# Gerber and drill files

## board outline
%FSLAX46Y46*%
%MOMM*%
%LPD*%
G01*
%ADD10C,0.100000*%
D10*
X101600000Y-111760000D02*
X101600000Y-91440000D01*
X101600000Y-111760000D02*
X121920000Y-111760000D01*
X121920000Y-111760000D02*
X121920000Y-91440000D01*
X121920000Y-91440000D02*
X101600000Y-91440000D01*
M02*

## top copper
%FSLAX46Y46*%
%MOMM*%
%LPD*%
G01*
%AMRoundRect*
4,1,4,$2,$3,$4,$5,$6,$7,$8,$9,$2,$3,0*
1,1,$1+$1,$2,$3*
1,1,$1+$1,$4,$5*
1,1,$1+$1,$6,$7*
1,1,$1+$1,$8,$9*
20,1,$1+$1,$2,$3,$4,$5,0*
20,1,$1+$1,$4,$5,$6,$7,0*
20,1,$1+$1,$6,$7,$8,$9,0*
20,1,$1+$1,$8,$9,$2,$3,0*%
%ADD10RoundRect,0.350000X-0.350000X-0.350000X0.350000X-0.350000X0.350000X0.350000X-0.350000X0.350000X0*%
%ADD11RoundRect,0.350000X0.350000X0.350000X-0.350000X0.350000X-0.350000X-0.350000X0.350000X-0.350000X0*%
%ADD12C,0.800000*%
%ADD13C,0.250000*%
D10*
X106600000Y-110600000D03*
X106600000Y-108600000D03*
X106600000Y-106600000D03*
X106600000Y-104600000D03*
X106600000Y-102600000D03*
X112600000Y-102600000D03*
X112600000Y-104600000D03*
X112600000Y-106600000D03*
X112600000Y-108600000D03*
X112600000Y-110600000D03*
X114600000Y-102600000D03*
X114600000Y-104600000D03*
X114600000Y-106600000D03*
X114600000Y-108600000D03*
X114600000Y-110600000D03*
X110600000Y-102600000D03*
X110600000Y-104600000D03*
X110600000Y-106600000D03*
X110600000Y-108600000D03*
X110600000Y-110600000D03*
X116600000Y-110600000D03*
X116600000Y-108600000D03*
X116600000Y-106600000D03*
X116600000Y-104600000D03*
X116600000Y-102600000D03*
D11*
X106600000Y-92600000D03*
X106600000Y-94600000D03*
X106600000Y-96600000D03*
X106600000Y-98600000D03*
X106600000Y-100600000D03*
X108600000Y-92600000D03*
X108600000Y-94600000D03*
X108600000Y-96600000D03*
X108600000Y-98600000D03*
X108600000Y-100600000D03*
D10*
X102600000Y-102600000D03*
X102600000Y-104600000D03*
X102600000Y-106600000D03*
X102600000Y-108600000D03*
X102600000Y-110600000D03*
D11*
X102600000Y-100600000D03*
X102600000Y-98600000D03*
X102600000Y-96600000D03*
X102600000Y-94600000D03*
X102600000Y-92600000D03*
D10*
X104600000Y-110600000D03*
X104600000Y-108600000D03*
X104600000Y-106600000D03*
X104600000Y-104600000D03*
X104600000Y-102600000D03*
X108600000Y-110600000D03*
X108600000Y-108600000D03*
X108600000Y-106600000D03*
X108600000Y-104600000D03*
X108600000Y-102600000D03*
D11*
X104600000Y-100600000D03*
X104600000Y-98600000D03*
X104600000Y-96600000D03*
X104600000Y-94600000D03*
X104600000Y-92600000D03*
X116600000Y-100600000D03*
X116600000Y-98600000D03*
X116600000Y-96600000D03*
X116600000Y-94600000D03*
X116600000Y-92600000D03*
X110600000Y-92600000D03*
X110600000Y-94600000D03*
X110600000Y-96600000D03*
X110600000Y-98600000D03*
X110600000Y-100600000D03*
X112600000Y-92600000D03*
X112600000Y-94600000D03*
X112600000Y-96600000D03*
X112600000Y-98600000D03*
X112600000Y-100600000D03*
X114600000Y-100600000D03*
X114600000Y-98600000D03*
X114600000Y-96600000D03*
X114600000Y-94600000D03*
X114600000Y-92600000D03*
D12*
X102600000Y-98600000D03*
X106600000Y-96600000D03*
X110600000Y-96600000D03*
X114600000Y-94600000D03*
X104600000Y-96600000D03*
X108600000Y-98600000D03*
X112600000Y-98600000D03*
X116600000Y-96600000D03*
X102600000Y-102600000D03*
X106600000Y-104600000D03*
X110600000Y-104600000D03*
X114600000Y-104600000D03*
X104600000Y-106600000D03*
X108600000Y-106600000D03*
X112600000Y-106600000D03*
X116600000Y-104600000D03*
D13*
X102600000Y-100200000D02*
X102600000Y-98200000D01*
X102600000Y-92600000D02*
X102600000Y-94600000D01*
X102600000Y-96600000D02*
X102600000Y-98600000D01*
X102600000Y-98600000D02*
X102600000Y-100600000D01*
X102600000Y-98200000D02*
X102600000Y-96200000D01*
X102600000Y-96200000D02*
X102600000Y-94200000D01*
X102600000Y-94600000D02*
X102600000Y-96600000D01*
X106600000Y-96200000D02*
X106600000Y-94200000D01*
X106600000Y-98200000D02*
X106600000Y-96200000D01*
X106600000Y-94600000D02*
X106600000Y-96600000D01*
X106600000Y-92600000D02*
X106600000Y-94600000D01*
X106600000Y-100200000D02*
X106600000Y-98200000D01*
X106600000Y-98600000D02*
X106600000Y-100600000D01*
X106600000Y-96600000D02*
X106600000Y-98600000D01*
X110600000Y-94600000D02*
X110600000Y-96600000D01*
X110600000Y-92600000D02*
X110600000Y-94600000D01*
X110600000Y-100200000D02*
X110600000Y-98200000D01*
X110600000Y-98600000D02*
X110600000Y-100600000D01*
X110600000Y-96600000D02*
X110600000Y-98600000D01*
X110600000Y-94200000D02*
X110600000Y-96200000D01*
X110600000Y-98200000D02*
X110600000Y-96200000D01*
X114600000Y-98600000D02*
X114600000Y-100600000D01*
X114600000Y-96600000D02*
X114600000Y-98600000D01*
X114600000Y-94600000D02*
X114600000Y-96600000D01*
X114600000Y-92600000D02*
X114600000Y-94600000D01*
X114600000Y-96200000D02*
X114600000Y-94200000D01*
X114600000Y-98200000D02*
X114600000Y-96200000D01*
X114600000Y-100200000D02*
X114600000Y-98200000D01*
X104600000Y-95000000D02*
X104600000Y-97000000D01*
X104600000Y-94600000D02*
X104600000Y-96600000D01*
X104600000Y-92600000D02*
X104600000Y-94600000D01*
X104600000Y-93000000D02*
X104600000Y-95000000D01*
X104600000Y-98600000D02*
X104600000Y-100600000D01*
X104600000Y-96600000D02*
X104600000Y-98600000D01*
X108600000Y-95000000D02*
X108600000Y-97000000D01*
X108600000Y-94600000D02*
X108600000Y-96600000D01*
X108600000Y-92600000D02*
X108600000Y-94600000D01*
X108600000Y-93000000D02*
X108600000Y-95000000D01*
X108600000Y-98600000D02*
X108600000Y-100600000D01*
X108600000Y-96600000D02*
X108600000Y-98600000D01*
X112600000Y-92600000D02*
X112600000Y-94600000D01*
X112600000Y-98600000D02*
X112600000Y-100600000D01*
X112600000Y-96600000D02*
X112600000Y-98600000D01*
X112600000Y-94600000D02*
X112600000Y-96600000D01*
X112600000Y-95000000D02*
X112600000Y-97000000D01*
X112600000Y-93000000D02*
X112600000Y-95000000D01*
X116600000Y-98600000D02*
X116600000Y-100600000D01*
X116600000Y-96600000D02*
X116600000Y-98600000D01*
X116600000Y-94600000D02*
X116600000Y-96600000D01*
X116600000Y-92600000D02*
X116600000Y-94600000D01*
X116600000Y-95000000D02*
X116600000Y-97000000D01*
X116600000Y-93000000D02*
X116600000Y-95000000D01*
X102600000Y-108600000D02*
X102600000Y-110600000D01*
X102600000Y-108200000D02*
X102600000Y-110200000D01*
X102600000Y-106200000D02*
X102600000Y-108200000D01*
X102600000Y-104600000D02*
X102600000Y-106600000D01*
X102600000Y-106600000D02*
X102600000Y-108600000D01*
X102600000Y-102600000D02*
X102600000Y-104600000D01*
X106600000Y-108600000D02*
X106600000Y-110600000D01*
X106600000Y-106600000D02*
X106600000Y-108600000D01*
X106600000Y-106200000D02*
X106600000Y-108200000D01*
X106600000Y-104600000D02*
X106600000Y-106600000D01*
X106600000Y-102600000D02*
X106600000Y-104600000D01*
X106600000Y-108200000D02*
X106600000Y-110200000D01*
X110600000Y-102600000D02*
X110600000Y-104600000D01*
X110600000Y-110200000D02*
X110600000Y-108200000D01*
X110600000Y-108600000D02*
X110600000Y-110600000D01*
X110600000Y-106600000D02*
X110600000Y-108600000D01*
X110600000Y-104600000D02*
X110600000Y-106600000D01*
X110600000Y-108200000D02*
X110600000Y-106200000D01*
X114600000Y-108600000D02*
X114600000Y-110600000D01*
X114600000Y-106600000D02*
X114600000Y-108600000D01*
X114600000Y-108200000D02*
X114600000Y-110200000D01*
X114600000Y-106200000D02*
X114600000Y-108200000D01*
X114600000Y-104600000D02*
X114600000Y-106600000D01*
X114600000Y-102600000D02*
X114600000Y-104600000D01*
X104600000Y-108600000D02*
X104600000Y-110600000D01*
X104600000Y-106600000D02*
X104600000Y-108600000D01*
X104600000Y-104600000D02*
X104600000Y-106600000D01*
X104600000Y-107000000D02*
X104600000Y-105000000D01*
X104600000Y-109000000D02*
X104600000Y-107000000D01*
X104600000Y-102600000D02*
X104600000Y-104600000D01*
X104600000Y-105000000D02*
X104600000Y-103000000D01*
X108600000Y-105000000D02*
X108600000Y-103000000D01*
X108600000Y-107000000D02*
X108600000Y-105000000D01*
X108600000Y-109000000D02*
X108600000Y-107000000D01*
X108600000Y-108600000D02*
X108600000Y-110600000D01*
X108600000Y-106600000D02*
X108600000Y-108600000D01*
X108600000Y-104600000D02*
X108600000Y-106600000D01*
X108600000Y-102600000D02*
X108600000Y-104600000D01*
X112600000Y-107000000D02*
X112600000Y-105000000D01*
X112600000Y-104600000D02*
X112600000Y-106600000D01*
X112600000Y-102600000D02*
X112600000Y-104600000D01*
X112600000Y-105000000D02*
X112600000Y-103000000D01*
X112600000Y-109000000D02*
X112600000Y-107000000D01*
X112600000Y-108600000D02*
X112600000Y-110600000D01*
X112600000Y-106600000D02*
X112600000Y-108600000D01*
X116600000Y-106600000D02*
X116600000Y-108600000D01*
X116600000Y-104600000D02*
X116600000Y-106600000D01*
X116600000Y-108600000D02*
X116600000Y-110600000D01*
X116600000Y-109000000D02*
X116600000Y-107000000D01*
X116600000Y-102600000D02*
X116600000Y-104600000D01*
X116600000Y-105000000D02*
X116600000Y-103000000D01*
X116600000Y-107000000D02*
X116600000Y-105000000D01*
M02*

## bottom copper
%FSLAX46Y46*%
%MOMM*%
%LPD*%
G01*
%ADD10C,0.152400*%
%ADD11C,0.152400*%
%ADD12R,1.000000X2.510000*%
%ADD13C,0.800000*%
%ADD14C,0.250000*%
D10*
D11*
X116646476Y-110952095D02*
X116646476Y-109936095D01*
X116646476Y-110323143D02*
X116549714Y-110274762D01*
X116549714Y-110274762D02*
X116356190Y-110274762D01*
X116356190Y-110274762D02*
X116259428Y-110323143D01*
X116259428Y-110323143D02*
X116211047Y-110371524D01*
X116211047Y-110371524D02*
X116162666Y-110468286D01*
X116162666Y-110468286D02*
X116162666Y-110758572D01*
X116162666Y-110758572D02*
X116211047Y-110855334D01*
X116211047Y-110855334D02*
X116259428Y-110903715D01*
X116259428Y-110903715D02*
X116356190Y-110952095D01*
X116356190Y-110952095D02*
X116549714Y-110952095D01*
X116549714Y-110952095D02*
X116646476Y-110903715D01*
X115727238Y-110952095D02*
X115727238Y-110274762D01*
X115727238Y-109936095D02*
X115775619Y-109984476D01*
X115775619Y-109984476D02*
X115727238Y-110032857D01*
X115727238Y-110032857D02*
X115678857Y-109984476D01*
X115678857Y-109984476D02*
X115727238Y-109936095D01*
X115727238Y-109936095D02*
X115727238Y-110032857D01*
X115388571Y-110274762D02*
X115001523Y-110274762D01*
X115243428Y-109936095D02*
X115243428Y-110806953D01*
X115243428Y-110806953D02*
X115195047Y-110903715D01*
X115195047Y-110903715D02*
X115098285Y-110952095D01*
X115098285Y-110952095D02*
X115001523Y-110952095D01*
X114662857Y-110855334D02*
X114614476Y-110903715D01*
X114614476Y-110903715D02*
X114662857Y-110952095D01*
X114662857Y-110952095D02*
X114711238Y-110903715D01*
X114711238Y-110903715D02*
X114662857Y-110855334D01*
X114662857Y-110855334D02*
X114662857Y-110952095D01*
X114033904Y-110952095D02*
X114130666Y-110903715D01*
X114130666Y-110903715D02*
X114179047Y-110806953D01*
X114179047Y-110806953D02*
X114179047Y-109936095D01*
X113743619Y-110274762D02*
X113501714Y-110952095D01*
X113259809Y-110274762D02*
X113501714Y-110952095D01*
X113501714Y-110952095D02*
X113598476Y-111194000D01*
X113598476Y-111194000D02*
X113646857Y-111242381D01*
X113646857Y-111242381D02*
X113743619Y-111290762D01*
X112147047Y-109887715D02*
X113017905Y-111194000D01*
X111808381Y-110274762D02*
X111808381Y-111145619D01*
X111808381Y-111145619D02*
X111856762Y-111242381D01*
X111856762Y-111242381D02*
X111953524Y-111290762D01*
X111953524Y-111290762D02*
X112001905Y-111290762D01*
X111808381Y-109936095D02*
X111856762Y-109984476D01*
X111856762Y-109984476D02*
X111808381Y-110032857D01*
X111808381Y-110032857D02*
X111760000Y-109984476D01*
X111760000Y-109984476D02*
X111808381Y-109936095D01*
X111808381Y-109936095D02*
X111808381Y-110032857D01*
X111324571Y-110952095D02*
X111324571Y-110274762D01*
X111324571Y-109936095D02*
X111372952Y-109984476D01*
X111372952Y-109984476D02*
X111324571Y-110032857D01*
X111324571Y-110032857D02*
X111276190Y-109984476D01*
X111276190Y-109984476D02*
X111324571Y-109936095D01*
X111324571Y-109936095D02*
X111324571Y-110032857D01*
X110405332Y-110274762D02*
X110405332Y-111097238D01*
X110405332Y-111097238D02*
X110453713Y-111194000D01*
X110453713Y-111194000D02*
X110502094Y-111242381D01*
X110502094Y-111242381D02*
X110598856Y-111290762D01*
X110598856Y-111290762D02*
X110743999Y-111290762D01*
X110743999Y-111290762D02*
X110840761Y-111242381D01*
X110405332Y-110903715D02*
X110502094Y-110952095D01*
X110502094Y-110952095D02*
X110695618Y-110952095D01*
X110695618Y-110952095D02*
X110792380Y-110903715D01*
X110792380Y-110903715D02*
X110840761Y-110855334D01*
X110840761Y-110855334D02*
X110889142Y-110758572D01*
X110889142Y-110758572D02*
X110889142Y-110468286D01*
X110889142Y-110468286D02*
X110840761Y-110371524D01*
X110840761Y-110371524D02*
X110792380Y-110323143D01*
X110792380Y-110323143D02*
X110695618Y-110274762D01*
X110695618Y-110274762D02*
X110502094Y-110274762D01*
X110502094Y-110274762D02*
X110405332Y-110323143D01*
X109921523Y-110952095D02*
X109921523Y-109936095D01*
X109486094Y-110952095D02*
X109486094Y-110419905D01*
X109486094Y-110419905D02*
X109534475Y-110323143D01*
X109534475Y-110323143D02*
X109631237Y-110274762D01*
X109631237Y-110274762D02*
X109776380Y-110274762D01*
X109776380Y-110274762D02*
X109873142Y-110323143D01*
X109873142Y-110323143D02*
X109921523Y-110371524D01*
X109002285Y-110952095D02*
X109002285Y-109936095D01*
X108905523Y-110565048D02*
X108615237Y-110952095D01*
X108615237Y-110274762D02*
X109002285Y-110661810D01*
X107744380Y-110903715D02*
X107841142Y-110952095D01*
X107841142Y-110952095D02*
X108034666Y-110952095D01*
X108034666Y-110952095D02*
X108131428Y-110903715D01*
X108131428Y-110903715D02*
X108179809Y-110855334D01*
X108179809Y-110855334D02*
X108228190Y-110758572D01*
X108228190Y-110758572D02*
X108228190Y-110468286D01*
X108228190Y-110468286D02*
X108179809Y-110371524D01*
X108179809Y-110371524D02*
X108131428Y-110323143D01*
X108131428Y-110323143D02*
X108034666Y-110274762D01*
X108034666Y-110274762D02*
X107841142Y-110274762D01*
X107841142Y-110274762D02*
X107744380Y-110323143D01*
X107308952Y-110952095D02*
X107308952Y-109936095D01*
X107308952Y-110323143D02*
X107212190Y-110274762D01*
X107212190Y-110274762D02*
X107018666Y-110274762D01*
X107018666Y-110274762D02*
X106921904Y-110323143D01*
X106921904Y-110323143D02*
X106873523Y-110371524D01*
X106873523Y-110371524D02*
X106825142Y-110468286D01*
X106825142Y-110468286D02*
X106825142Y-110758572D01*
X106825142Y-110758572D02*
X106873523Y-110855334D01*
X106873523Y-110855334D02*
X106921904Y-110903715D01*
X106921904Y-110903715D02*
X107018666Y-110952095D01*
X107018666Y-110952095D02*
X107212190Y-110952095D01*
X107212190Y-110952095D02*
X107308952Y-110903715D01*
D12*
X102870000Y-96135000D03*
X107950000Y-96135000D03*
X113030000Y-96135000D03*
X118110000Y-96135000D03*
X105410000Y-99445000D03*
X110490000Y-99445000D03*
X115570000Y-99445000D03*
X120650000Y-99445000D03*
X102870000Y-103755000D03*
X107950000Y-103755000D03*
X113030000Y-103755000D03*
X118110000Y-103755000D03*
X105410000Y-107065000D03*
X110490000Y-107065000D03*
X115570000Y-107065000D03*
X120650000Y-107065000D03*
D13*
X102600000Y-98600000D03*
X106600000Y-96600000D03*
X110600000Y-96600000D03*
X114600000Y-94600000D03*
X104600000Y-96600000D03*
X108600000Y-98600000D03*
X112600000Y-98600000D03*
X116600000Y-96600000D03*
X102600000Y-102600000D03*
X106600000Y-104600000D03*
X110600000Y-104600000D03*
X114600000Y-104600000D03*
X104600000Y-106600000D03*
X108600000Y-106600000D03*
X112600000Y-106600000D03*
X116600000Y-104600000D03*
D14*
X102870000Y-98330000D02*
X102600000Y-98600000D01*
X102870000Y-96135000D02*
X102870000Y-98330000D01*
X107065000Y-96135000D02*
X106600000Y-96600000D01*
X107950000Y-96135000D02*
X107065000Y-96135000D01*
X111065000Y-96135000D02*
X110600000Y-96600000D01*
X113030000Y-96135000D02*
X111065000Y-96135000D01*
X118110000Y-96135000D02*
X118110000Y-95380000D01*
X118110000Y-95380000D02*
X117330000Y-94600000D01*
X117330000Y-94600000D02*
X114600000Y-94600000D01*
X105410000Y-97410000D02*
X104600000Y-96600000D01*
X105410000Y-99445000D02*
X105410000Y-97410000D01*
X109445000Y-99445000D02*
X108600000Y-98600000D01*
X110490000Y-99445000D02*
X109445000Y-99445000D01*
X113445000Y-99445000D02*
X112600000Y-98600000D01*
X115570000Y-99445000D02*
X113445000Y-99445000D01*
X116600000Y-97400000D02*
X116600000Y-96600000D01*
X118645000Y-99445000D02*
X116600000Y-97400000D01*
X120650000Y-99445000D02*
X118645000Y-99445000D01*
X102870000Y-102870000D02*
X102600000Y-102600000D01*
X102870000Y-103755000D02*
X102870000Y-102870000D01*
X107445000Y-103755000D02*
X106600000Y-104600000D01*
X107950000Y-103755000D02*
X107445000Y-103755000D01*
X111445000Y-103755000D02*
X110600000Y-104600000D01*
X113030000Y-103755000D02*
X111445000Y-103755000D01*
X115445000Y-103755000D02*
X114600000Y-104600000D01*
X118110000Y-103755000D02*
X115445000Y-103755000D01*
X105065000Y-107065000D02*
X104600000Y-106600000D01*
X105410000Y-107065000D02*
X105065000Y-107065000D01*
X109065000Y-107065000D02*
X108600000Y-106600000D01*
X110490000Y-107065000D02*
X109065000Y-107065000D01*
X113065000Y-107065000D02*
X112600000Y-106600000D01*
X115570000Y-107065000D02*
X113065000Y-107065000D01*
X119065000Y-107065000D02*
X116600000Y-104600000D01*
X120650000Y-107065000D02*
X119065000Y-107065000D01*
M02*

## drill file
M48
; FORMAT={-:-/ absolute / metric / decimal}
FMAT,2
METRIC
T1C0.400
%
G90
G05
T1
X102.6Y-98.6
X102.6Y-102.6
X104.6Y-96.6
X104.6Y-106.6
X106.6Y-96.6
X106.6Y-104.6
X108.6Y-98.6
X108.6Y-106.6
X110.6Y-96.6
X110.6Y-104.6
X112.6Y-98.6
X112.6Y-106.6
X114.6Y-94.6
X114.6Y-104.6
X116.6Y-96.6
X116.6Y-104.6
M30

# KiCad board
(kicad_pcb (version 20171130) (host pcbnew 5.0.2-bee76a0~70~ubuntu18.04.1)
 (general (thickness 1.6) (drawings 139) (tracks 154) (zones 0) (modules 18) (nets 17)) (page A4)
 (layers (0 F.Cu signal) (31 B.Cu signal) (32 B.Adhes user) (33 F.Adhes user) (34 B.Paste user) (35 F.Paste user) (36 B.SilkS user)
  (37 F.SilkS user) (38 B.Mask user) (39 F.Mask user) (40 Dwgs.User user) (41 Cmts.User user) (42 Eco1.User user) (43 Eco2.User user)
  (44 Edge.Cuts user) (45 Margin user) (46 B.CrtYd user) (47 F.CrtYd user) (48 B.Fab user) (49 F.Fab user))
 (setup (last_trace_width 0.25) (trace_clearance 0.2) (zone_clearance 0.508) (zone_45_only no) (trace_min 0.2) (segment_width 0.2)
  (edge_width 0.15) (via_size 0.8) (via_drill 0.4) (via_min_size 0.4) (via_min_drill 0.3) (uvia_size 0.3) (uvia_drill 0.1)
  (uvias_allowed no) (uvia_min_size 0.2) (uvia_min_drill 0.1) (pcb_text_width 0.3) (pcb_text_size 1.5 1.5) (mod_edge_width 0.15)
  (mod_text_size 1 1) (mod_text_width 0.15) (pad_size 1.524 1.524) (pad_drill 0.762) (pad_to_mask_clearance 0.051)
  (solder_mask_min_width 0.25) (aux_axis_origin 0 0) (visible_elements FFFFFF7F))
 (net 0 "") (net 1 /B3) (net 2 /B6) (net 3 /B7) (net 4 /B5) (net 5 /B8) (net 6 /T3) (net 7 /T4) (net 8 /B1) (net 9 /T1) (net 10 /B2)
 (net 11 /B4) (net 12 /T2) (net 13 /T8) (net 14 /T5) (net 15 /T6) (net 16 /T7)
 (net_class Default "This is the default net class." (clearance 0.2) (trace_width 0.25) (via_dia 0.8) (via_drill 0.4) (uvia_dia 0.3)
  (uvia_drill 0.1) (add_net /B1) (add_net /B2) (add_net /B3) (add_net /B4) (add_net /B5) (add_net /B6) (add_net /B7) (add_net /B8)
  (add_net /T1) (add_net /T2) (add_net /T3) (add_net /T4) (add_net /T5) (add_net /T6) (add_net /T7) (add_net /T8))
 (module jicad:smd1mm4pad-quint (layer F.Cu) (at 106.6 102.6)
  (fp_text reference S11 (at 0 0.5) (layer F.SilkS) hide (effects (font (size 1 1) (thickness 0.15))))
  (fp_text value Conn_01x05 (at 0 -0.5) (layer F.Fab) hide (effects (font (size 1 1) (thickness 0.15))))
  (pad 5 smd roundrect (at 0 8) (size 1.4 1.4) (layers F.Cu F.Paste F.Mask) (roundrect_rratio 0.25) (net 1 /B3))
  (pad 4 smd roundrect (at 0 6) (size 1.4 1.4) (layers F.Cu F.Paste F.Mask) (roundrect_rratio 0.25) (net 1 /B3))
  (pad 3 smd roundrect (at 0 4) (size 1.4 1.4) (layers F.Cu F.Paste F.Mask) (roundrect_rratio 0.25) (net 1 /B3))
  (pad 2 smd roundrect (at 0 2) (size 1.4 1.4) (layers F.Cu F.Paste F.Mask) (roundrect_rratio 0.25) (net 1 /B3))
  (pad 1 smd roundrect (at 0 0) (size 1.4 1.4) (layers F.Cu F.Paste F.Mask) (roundrect_rratio 0.25) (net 1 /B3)))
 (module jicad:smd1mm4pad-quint (layer F.Cu) (at 112.6 102.6)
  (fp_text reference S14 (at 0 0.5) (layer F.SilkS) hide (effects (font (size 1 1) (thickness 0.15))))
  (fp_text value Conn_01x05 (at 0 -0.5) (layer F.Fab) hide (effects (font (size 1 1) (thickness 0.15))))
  (pad 1 smd roundrect (at 0 0) (size 1.4 1.4) (layers F.Cu F.Paste F.Mask) (roundrect_rratio 0.25) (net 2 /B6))
  (pad 2 smd roundrect (at 0 2) (size 1.4 1.4) (layers F.Cu F.Paste F.Mask) (roundrect_rratio 0.25) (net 2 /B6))
  (pad 3 smd roundrect (at 0 4) (size 1.4 1.4) (layers F.Cu F.Paste F.Mask) (roundrect_rratio 0.25) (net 2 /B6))
  (pad 4 smd roundrect (at 0 6) (size 1.4 1.4) (layers F.Cu F.Paste F.Mask) (roundrect_rratio 0.25) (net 2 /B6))
  (pad 5 smd roundrect (at 0 8) (size 1.4 1.4) (layers F.Cu F.Paste F.Mask) (roundrect_rratio 0.25) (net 2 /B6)))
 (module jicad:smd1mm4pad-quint (layer F.Cu) (at 114.6 102.6)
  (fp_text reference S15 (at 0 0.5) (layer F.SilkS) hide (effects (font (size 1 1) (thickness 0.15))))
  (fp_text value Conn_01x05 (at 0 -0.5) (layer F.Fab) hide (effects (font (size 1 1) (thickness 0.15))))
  (pad 1 smd roundrect (at 0 0) (size 1.4 1.4) (layers F.Cu F.Paste F.Mask) (roundrect_rratio 0.25) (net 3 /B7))
  (pad 2 smd roundrect (at 0 2) (size 1.4 1.4) (layers F.Cu F.Paste F.Mask) (roundrect_rratio 0.25) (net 3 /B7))
  (pad 3 smd roundrect (at 0 4) (size 1.4 1.4) (layers F.Cu F.Paste F.Mask) (roundrect_rratio 0.25) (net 3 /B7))
  (pad 4 smd roundrect (at 0 6) (size 1.4 1.4) (layers F.Cu F.Paste F.Mask) (roundrect_rratio 0.25) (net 3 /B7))
  (pad 5 smd roundrect (at 0 8) (size 1.4 1.4) (layers F.Cu F.Paste F.Mask) (roundrect_rratio 0.25) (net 3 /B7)))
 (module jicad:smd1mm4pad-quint (layer F.Cu) (at 110.6 102.6)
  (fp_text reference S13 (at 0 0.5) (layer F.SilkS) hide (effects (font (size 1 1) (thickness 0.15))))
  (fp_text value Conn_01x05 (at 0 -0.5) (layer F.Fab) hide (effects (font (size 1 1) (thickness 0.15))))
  (pad 1 smd roundrect (at 0 0) (size 1.4 1.4) (layers F.Cu F.Paste F.Mask) (roundrect_rratio 0.25) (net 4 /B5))
  (pad 2 smd roundrect (at 0 2) (size 1.4 1.4) (layers F.Cu F.Paste F.Mask) (roundrect_rratio 0.25) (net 4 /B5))
  (pad 3 smd roundrect (at 0 4) (size 1.4 1.4) (layers F.Cu F.Paste F.Mask) (roundrect_rratio 0.25) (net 4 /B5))
  (pad 4 smd roundrect (at 0 6) (size 1.4 1.4) (layers F.Cu F.Paste F.Mask) (roundrect_rratio 0.25) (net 4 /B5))
  (pad 5 smd roundrect (at 0 8) (size 1.4 1.4) (layers F.Cu F.Paste F.Mask) (roundrect_rratio 0.25) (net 4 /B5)))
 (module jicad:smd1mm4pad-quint (layer F.Cu) (at 116.6 102.6)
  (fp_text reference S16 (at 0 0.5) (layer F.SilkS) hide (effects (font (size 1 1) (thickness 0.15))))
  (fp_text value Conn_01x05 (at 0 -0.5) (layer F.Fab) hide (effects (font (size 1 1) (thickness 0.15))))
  (pad 5 smd roundrect (at 0 8) (size 1.4 1.4) (layers F.Cu F.Paste F.Mask) (roundrect_rratio 0.25) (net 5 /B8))
  (pad 4 smd roundrect (at 0 6) (size 1.4 1.4) (layers F.Cu F.Paste F.Mask) (roundrect_rratio 0.25) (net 5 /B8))
  (pad 3 smd roundrect (at 0 4) (size 1.4 1.4) (layers F.Cu F.Paste F.Mask) (roundrect_rratio 0.25) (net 5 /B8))
  (pad 2 smd roundrect (at 0 2) (size 1.4 1.4) (layers F.Cu F.Paste F.Mask) (roundrect_rratio 0.25) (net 5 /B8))
  (pad 1 smd roundrect (at 0 0) (size 1.4 1.4) (layers F.Cu F.Paste F.Mask) (roundrect_rratio 0.25) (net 5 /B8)))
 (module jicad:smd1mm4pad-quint (layer F.Cu) (at 106.6 100.6 180)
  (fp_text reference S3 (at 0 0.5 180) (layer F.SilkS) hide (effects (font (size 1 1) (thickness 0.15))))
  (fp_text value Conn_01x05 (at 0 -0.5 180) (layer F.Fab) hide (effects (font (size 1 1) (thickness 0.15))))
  (pad 5 smd roundrect (at 0 8 180) (size 1.4 1.4) (layers F.Cu F.Paste F.Mask) (roundrect_rratio 0.25) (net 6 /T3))
  (pad 4 smd roundrect (at 0 6 180) (size 1.4 1.4) (layers F.Cu F.Paste F.Mask) (roundrect_rratio 0.25) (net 6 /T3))
  (pad 3 smd roundrect (at 0 4 180) (size 1.4 1.4) (layers F.Cu F.Paste F.Mask) (roundrect_rratio 0.25) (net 6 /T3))
  (pad 2 smd roundrect (at 0 2 180) (size 1.4 1.4) (layers F.Cu F.Paste F.Mask) (roundrect_rratio 0.25) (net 6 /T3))
  (pad 1 smd roundrect (at 0 0 180) (size 1.4 1.4) (layers F.Cu F.Paste F.Mask) (roundrect_rratio 0.25) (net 6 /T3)))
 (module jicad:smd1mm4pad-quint (layer F.Cu) (at 108.6 100.6 180)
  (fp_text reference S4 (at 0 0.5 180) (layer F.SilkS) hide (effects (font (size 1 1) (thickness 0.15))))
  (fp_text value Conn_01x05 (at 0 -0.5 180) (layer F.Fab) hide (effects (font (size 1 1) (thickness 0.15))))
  (pad 5 smd roundrect (at 0 8 180) (size 1.4 1.4) (layers F.Cu F.Paste F.Mask) (roundrect_rratio 0.25) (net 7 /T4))
  (pad 4 smd roundrect (at 0 6 180) (size 1.4 1.4) (layers F.Cu F.Paste F.Mask) (roundrect_rratio 0.25) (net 7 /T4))
  (pad 3 smd roundrect (at 0 4 180) (size 1.4 1.4) (layers F.Cu F.Paste F.Mask) (roundrect_rratio 0.25) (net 7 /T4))
  (pad 2 smd roundrect (at 0 2 180) (size 1.4 1.4) (layers F.Cu F.Paste F.Mask) (roundrect_rratio 0.25) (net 7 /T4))
  (pad 1 smd roundrect (at 0 0 180) (size 1.4 1.4) (layers F.Cu F.Paste F.Mask) (roundrect_rratio 0.25) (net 7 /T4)))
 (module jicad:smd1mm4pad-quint (layer F.Cu) (at 102.6 102.6)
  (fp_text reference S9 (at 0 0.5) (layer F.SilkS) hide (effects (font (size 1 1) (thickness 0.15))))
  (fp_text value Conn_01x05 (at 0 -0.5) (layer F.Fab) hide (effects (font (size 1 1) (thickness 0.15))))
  (pad 1 smd roundrect (at 0 0) (size 1.4 1.4) (layers F.Cu F.Paste F.Mask) (roundrect_rratio 0.25) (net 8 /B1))
  (pad 2 smd roundrect (at 0 2) (size 1.4 1.4) (layers F.Cu F.Paste F.Mask) (roundrect_rratio 0.25) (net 8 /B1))
  (pad 3 smd roundrect (at 0 4) (size 1.4 1.4) (layers F.Cu F.Paste F.Mask) (roundrect_rratio 0.25) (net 8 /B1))
  (pad 4 smd roundrect (at 0 6) (size 1.4 1.4) (layers F.Cu F.Paste F.Mask) (roundrect_rratio 0.25) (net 8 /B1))
  (pad 5 smd roundrect (at 0 8) (size 1.4 1.4) (layers F.Cu F.Paste F.Mask) (roundrect_rratio 0.25) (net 8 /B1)))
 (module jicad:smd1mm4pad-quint (layer F.Cu) (at 102.6 100.6 180)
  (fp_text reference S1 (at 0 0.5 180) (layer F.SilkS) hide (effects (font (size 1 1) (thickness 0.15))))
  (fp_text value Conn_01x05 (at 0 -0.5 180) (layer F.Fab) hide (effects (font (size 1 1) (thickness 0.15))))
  (pad 1 smd roundrect (at 0 0 180) (size 1.4 1.4) (layers F.Cu F.Paste F.Mask) (roundrect_rratio 0.25) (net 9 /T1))
  (pad 2 smd roundrect (at 0 2 180) (size 1.4 1.4) (layers F.Cu F.Paste F.Mask) (roundrect_rratio 0.25) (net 9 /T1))
  (pad 3 smd roundrect (at 0 4 180) (size 1.4 1.4) (layers F.Cu F.Paste F.Mask) (roundrect_rratio 0.25) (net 9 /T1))
  (pad 4 smd roundrect (at 0 6 180) (size 1.4 1.4) (layers F.Cu F.Paste F.Mask) (roundrect_rratio 0.25) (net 9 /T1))
  (pad 5 smd roundrect (at 0 8 180) (size 1.4 1.4) (layers F.Cu F.Paste F.Mask) (roundrect_rratio 0.25) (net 9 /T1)))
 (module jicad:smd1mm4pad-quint (layer F.Cu) (at 104.6 102.6)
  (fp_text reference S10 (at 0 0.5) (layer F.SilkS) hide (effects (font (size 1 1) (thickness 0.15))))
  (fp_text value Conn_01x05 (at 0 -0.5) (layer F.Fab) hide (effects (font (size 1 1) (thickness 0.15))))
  (pad 5 smd roundrect (at 0 8) (size 1.4 1.4) (layers F.Cu F.Paste F.Mask) (roundrect_rratio 0.25) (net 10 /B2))
  (pad 4 smd roundrect (at 0 6) (size 1.4 1.4) (layers F.Cu F.Paste F.Mask) (roundrect_rratio 0.25) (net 10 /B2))
  (pad 3 smd roundrect (at 0 4) (size 1.4 1.4) (layers F.Cu F.Paste F.Mask) (roundrect_rratio 0.25) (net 10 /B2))
  (pad 2 smd roundrect (at 0 2) (size 1.4 1.4) (layers F.Cu F.Paste F.Mask) (roundrect_rratio 0.25) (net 10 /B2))
  (pad 1 smd roundrect (at 0 0) (size 1.4 1.4) (layers F.Cu F.Paste F.Mask) (roundrect_rratio 0.25) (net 10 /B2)))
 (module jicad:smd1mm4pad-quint (layer F.Cu) (at 108.6 102.6)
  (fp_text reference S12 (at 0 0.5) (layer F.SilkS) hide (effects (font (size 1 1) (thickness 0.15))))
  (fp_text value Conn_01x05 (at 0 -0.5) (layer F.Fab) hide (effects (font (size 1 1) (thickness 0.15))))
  (pad 5 smd roundrect (at 0 8) (size 1.4 1.4) (layers F.Cu F.Paste F.Mask) (roundrect_rratio 0.25) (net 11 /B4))
  (pad 4 smd roundrect (at 0 6) (size 1.4 1.4) (layers F.Cu F.Paste F.Mask) (roundrect_rratio 0.25) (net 11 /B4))
  (pad 3 smd roundrect (at 0 4) (size 1.4 1.4) (layers F.Cu F.Paste F.Mask) (roundrect_rratio 0.25) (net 11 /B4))
  (pad 2 smd roundrect (at 0 2) (size 1.4 1.4) (layers F.Cu F.Paste F.Mask) (roundrect_rratio 0.25) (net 11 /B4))
  (pad 1 smd roundrect (at 0 0) (size 1.4 1.4) (layers F.Cu F.Paste F.Mask) (roundrect_rratio 0.25) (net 11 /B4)))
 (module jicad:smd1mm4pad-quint (layer F.Cu) (at 104.6 100.6 180)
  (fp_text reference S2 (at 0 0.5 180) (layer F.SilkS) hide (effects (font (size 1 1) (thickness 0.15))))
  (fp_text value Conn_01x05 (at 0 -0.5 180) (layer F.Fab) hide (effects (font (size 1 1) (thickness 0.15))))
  (pad 1 smd roundrect (at 0 0 180) (size 1.4 1.4) (layers F.Cu F.Paste F.Mask) (roundrect_rratio 0.25) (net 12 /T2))
  (pad 2 smd roundrect (at 0 2 180) (size 1.4 1.4) (layers F.Cu F.Paste F.Mask) (roundrect_rratio 0.25) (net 12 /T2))
  (pad 3 smd roundrect (at 0 4 180) (size 1.4 1.4) (layers F.Cu F.Paste F.Mask) (roundrect_rratio 0.25) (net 12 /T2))
  (pad 4 smd roundrect (at 0 6 180) (size 1.4 1.4) (layers F.Cu F.Paste F.Mask) (roundrect_rratio 0.25) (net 12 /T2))
  (pad 5 smd roundrect (at 0 8 180) (size 1.4 1.4) (layers F.Cu F.Paste F.Mask) (roundrect_rratio 0.25) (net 12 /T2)))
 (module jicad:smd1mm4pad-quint (layer F.Cu) (at 116.6 100.6 180)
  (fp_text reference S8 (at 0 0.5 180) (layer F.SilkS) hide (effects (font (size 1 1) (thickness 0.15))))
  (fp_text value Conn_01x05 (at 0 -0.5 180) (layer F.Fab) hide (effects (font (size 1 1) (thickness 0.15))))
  (pad 1 smd roundrect (at 0 0 180) (size 1.4 1.4) (layers F.Cu F.Paste F.Mask) (roundrect_rratio 0.25) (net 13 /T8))
  (pad 2 smd roundrect (at 0 2 180) (size 1.4 1.4) (layers F.Cu F.Paste F.Mask) (roundrect_rratio 0.25) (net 13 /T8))
  (pad 3 smd roundrect (at 0 4 180) (size 1.4 1.4) (layers F.Cu F.Paste F.Mask) (roundrect_rratio 0.25) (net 13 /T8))
  (pad 4 smd roundrect (at 0 6 180) (size 1.4 1.4) (layers F.Cu F.Paste F.Mask) (roundrect_rratio 0.25) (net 13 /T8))
  (pad 5 smd roundrect (at 0 8 180) (size 1.4 1.4) (layers F.Cu F.Paste F.Mask) (roundrect_rratio 0.25) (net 13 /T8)))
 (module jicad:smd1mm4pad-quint (layer F.Cu) (at 110.6 100.6 180)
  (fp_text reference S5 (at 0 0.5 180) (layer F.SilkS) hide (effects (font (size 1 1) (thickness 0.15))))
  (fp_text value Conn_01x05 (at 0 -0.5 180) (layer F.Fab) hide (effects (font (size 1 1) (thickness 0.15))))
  (pad 5 smd roundrect (at 0 8 180) (size 1.4 1.4) (layers F.Cu F.Paste F.Mask) (roundrect_rratio 0.25) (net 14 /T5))
  (pad 4 smd roundrect (at 0 6 180) (size 1.4 1.4) (layers F.Cu F.Paste F.Mask) (roundrect_rratio 0.25) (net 14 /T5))
  (pad 3 smd roundrect (at 0 4 180) (size 1.4 1.4) (layers F.Cu F.Paste F.Mask) (roundrect_rratio 0.25) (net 14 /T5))
  (pad 2 smd roundrect (at 0 2 180) (size 1.4 1.4) (layers F.Cu F.Paste F.Mask) (roundrect_rratio 0.25) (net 14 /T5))
  (pad 1 smd roundrect (at 0 0 180) (size 1.4 1.4) (layers F.Cu F.Paste F.Mask) (roundrect_rratio 0.25) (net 14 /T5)))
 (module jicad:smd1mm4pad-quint (layer F.Cu) (at 112.6 100.6 180)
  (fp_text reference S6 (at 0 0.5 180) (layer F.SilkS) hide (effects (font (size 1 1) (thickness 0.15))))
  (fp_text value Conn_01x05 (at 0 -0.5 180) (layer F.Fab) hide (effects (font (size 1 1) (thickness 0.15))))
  (pad 5 smd roundrect (at 0 8 180) (size 1.4 1.4) (layers F.Cu F.Paste F.Mask) (roundrect_rratio 0.25) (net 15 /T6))
  (pad 4 smd roundrect (at 0 6 180) (size 1.4 1.4) (layers F.Cu F.Paste F.Mask) (roundrect_rratio 0.25) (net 15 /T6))
  (pad 3 smd roundrect (at 0 4 180) (size 1.4 1.4) (layers F.Cu F.Paste F.Mask) (roundrect_rratio 0.25) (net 15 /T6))
  (pad 2 smd roundrect (at 0 2 180) (size 1.4 1.4) (layers F.Cu F.Paste F.Mask) (roundrect_rratio 0.25) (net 15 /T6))
  (pad 1 smd roundrect (at 0 0 180) (size 1.4 1.4) (layers F.Cu F.Paste F.Mask) (roundrect_rratio 0.25) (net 15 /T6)))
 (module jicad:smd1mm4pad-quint (layer F.Cu) (at 114.6 100.6 180)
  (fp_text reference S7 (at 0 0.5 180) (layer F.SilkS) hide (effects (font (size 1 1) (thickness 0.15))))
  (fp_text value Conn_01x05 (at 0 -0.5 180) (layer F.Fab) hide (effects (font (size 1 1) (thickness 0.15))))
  (pad 1 smd roundrect (at 0 0 180) (size 1.4 1.4) (layers F.Cu F.Paste F.Mask) (roundrect_rratio 0.25) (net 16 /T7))
  (pad 2 smd roundrect (at 0 2 180) (size 1.4 1.4) (layers F.Cu F.Paste F.Mask) (roundrect_rratio 0.25) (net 16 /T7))
  (pad 3 smd roundrect (at 0 4 180) (size 1.4 1.4) (layers F.Cu F.Paste F.Mask) (roundrect_rratio 0.25) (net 16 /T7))
  (pad 4 smd roundrect (at 0 6 180) (size 1.4 1.4) (layers F.Cu F.Paste F.Mask) (roundrect_rratio 0.25) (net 16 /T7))
  (pad 5 smd roundrect (at 0 8 180) (size 1.4 1.4) (layers F.Cu F.Paste F.Mask) (roundrect_rratio 0.25) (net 16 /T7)))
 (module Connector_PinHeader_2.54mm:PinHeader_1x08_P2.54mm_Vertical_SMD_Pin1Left (layer B.Cu) (at 111.76 97.79 270)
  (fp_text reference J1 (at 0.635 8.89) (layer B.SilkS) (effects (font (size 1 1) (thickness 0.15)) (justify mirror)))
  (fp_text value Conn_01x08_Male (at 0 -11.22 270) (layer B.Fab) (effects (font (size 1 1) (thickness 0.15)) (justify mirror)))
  (pad 1 smd rect (at -1.655 8.89 270) (size 2.51 1) (layers B.Cu B.Paste B.Mask) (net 9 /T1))
  (pad 3 smd rect (at -1.655 3.81 270) (size 2.51 1) (layers B.Cu B.Paste B.Mask) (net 6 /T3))
  (pad 5 smd rect (at -1.655 -1.27 270) (size 2.51 1) (layers B.Cu B.Paste B.Mask) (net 14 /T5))
  (pad 7 smd rect (at -1.655 -6.35 270) (size 2.51 1) (layers B.Cu B.Paste B.Mask) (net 16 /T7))
  (pad 2 smd rect (at 1.655 6.35 270) (size 2.51 1) (layers B.Cu B.Paste B.Mask) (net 12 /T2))
  (pad 4 smd rect (at 1.655 1.27 270) (size 2.51 1) (layers B.Cu B.Paste B.Mask) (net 7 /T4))
  (pad 6 smd rect (at 1.655 -3.81 270) (size 2.51 1) (layers B.Cu B.Paste B.Mask) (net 15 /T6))
  (pad 8 smd rect (at 1.655 -8.89 270) (size 2.51 1) (layers B.Cu B.Paste B.Mask) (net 13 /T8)))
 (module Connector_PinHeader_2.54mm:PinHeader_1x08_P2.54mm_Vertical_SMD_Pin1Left (layer B.Cu) (at 111.76 105.41 270)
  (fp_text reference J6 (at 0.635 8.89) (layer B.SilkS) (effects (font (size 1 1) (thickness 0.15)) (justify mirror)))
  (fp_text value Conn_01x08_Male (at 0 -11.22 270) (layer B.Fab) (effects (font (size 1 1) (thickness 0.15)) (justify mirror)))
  (pad 1 smd rect (at -1.655 8.89 270) (size 2.51 1) (layers B.Cu B.Paste B.Mask) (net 8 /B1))
  (pad 3 smd rect (at -1.655 3.81 270) (size 2.51 1) (layers B.Cu B.Paste B.Mask) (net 1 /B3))
  (pad 5 smd rect (at -1.655 -1.27 270) (size 2.51 1) (layers B.Cu B.Paste B.Mask) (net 4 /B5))
  (pad 7 smd rect (at -1.655 -6.35 270) (size 2.51 1) (layers B.Cu B.Paste B.Mask) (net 3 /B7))
  (pad 2 smd rect (at 1.655 6.35 270) (size 2.51 1) (layers B.Cu B.Paste B.Mask) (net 10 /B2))
  (pad 4 smd rect (at 1.655 1.27 270) (size 2.51 1) (layers B.Cu B.Paste B.Mask) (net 11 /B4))
  (pad 6 smd rect (at 1.655 -3.81 270) (size 2.51 1) (layers B.Cu B.Paste B.Mask) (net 2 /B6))
  (pad 8 smd rect (at 1.655 -8.89 270) (size 2.51 1) (layers B.Cu B.Paste B.Mask) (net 5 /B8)))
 (gr_line (start 101.6 111.76) (end 101.6 91.44) (layer Edge.Cuts) (width 0.1))
 (gr_line (start 101.6 111.76) (end 121.92 111.76) (layer Edge.Cuts) (width 0.1))
 (gr_line (start 121.92 111.76) (end 121.92 91.44) (layer Edge.Cuts) (width 0.1))
 (gr_line (start 121.92 91.44) (end 101.6 91.44) (layer Edge.Cuts) (width 0.1))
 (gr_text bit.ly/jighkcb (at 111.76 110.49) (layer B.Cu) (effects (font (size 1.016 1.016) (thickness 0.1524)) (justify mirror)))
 (segment (start 102.6 100.2) (end 102.6 98.2) (width 0.25) (layer F.Cu) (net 9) (status 30))
 (segment (start 102.6 92.6) (end 102.6 94.6) (width 0.25) (layer F.Cu) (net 9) (status 30))
 (segment (start 102.6 96.6) (end 102.6 98.6) (width 0.25) (layer F.Cu) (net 9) (status 30))
 (segment (start 102.6 98.6) (end 102.6 100.6) (width 0.25) (layer F.Cu) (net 9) (status 30))
 (segment (start 102.6 98.2) (end 102.6 96.2) (width 0.25) (layer F.Cu) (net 9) (status 30))
 (segment (start 102.6 96.2) (end 102.6 94.2) (width 0.25) (layer F.Cu) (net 9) (status 30))
 (segment (start 102.6 94.6) (end 102.6 96.6) (width 0.25) (layer F.Cu) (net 9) (status 30))
 (via (at 102.6 98.6) (size 0.8) (drill 0.4) (layers F.Cu B.Cu) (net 9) (status 30))
 (segment (start 102.87 98.33) (end 102.6 98.6) (width 0.25) (layer B.Cu) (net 9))
 (segment (start 102.87 96.135) (end 102.87 98.33) (width 0.25) (layer B.Cu) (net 9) (status 10))
 (segment (start 106.6 96.2) (end 106.6 94.2) (width 0.25) (layer F.Cu) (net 6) (status 30))
 (segment (start 106.6 98.2) (end 106.6 96.2) (width 0.25) (layer F.Cu) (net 6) (status 30))
 (segment (start 106.6 94.6) (end 106.6 96.6) (width 0.25) (layer F.Cu) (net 6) (status 30))
 (segment (start 106.6 92.6) (end 106.6 94.6) (width 0.25) (layer F.Cu) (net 6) (status 30))
 (segment (start 106.6 100.2) (end 106.6 98.2) (width 0.25) (layer F.Cu) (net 6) (status 30))
 (segment (start 106.6 98.6) (end 106.6 100.6) (width 0.25) (layer F.Cu) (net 6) (status 30))
 (segment (start 106.6 96.6) (end 106.6 98.6) (width 0.25) (layer F.Cu) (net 6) (status 30))
 (via (at 106.6 96.6) (size 0.8) (drill 0.4) (layers F.Cu B.Cu) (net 6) (status 30))
 (segment (start 107.065 96.135) (end 106.6 96.6) (width 0.25) (layer B.Cu) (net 6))
 (segment (start 107.95 96.135) (end 107.065 96.135) (width 0.25) (layer B.Cu) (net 6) (status 10))
 (segment (start 110.6 94.6) (end 110.6 96.6) (width 0.25) (layer F.Cu) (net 14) (status 30))
 (segment (start 110.6 92.6) (end 110.6 94.6) (width 0.25) (layer F.Cu) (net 14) (status 30))
 (segment (start 110.6 100.2) (end 110.6 98.2) (width 0.25) (layer F.Cu) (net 14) (status 30))
 (segment (start 110.6 98.6) (end 110.6 100.6) (width 0.25) (layer F.Cu) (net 14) (status 30))
 (segment (start 110.6 96.6) (end 110.6 98.6) (width 0.25) (layer F.Cu) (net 14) (status 30))
 (segment (start 110.6 94.2) (end 110.6 96.2) (width 0.25) (layer F.Cu) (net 14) (status 30))
 (segment (start 110.6 98.2) (end 110.6 96.2) (width 0.25) (layer F.Cu) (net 14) (status 30))
 (via (at 110.6 96.6) (size 0.8) (drill 0.4) (layers F.Cu B.Cu) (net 14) (status 30))
 (segment (start 111.065 96.135) (end 110.6 96.6) (width 0.25) (layer B.Cu) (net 14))
 (segment (start 113.03 96.135) (end 111.065 96.135) (width 0.25) (layer B.Cu) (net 14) (status 10))
 (segment (start 114.6 98.6) (end 114.6 100.6) (width 0.25) (layer F.Cu) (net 16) (status 30))
 (segment (start 114.6 96.6) (end 114.6 98.6) (width 0.25) (layer F.Cu) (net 16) (status 30))
 (segment (start 114.6 94.6) (end 114.6 96.6) (width 0.25) (layer F.Cu) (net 16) (status 30))
 (segment (start 114.6 92.6) (end 114.6 94.6) (width 0.25) (layer F.Cu) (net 16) (status 30))
 (segment (start 114.6 96.2) (end 114.6 94.2) (width 0.25) (layer F.Cu) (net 16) (status 30))
 (segment (start 114.6 98.2) (end 114.6 96.2) (width 0.25) (layer F.Cu) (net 16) (status 30))
 (segment (start 114.6 100.2) (end 114.6 98.2) (width 0.25) (layer F.Cu) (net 16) (status 30))
 (segment (start 118.11 96.135) (end 118.11 95.38) (width 0.25) (layer B.Cu) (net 16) (status 30))
 (segment (start 118.11 95.38) (end 117.33 94.6) (width 0.25) (layer B.Cu) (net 16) (status 10))
 (via (at 114.6 94.6) (size 0.8) (drill 0.4) (layers F.Cu B.Cu) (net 16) (status 30))
 (segment (start 117.33 94.6) (end 114.6 94.6) (width 0.25) (layer B.Cu) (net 16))
 (segment (start 104.6 95) (end 104.6 97) (width 0.25) (layer F.Cu) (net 12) (status 30))
 (segment (start 104.6 94.6) (end 104.6 96.6) (width 0.25) (layer F.Cu) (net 12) (status 30))
 (segment (start 104.6 92.6) (end 104.6 94.6) (width 0.25) (layer F.Cu) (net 12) (status 30))
 (segment (start 104.6 93) (end 104.6 95) (width 0.25) (layer F.Cu) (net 12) (status 30))
 (segment (start 104.6 98.6) (end 104.6 100.6) (width 0.25) (layer F.Cu) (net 12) (status 30))
 (segment (start 104.6 96.6) (end 104.6 98.6) (width 0.25) (layer F.Cu) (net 12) (status 30))
 (via (at 104.6 96.6) (size 0.8) (drill 0.4) (layers F.Cu B.Cu) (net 12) (status 30))
 (segment (start 105.41 97.41) (end 104.6 96.6) (width 0.25) (layer B.Cu) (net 12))
 (segment (start 105.41 99.445) (end 105.41 97.41) (width 0.25) (layer B.Cu) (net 12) (status 10))
 (segment (start 108.6 95) (end 108.6 97) (width 0.25) (layer F.Cu) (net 7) (status 30))
 (segment (start 108.6 94.6) (end 108.6 96.6) (width 0.25) (layer F.Cu) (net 7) (status 30))
 (segment (start 108.6 92.6) (end 108.6 94.6) (width 0.25) (layer F.Cu) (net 7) (status 30))
 (segment (start 108.6 93) (end 108.6 95) (width 0.25) (layer F.Cu) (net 7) (status 30))
 (segment (start 108.6 98.6) (end 108.6 100.6) (width 0.25) (layer F.Cu) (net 7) (status 30))
 (segment (start 108.6 96.6) (end 108.6 98.6) (width 0.25) (layer F.Cu) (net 7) (status 30))
 (via (at 108.6 98.6) (size 0.8) (drill 0.4) (layers F.Cu B.Cu) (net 7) (status 30))
 (segment (start 109.445 99.445) (end 108.6 98.6) (width 0.25) (layer B.Cu) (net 7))
 (segment (start 110.49 99.445) (end 109.445 99.445) (width 0.25) (layer B.Cu) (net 7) (status 10))
 (segment (start 112.6 92.6) (end 112.6 94.6) (width 0.25) (layer F.Cu) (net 15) (status 30))
 (segment (start 112.6 98.6) (end 112.6 100.6) (width 0.25) (layer F.Cu) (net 15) (status 30))
 (segment (start 112.6 96.6) (end 112.6 98.6) (width 0.25) (layer F.Cu) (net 15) (status 30))
 (segment (start 112.6 94.6) (end 112.6 96.6) (width 0.25) (layer F.Cu) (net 15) (status 30))
 (segment (start 112.6 95) (end 112.6 97) (width 0.25) (layer F.Cu) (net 15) (status 30))
 (segment (start 112.6 93) (end 112.6 95) (width 0.25) (layer F.Cu) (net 15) (status 30))
 (via (at 112.6 98.6) (size 0.8) (drill 0.4) (layers F.Cu B.Cu) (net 15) (status 30))
 (segment (start 113.445 99.445) (end 112.6 98.6) (width 0.25) (layer B.Cu) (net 15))
 (segment (start 115.57 99.445) (end 113.445 99.445) (width 0.25) (layer B.Cu) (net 15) (status 10))
 (segment (start 116.6 98.6) (end 116.6 100.6) (width 0.25) (layer F.Cu) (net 13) (status 30))
 (segment (start 116.6 96.6) (end 116.6 98.6) (width 0.25) (layer F.Cu) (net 13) (status 30))
 (segment (start 116.6 94.6) (end 116.6 96.6) (width 0.25) (layer F.Cu) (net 13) (status 30))
 (segment (start 116.6 92.6) (end 116.6 94.6) (width 0.25) (layer F.Cu) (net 13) (status 30))
 (segment (start 116.6 95) (end 116.6 97) (width 0.25) (layer F.Cu) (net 13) (status 30))
 (segment (start 116.6 93) (end 116.6 95) (width 0.25) (layer F.Cu) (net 13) (status 30))
 (via (at 116.6 96.6) (size 0.8) (drill 0.4) (layers F.Cu B.Cu) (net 13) (status 30))
 (segment (start 116.6 97.4) (end 116.6 96.6) (width 0.25) (layer B.Cu) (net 13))
 (segment (start 118.645 99.445) (end 116.6 97.4) (width 0.25) (layer B.Cu) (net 13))
 (segment (start 120.65 99.445) (end 118.645 99.445) (width 0.25) (layer B.Cu) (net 13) (status 10))
 (segment (start 102.6 108.6) (end 102.6 110.6) (width 0.25) (layer F.Cu) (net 8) (status 30))
 (segment (start 102.6 108.2) (end 102.6 110.2) (width 0.25) (layer F.Cu) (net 8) (status 30))
 (segment (start 102.6 106.2) (end 102.6 108.2) (width 0.25) (layer F.Cu) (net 8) (status 30))
 (segment (start 102.6 104.6) (end 102.6 106.6) (width 0.25) (layer F.Cu) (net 8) (status 30))
 (segment (start 102.6 106.6) (end 102.6 108.6) (width 0.25) (layer F.Cu) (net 8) (status 30))
 (segment (start 102.6 102.6) (end 102.6 104.6) (width 0.25) (layer F.Cu) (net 8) (status 30))
 (via (at 102.6 102.6) (size 0.8) (drill 0.4) (layers F.Cu B.Cu) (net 8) (status 30))
 (segment (start 102.87 102.87) (end 102.6 102.6) (width 0.25) (layer B.Cu) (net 8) (status 30))
 (segment (start 102.87 103.755) (end 102.87 102.87) (width 0.25) (layer B.Cu) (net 8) (status 30))
 (segment (start 106.6 108.6) (end 106.6 110.6) (width 0.25) (layer F.Cu) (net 1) (status 30))
 (segment (start 106.6 106.6) (end 106.6 108.6) (width 0.25) (layer F.Cu) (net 1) (status 30))
 (segment (start 106.6 106.2) (end 106.6 108.2) (width 0.25) (layer F.Cu) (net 1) (status 30))
 (segment (start 106.6 104.6) (end 106.6 106.6) (width 0.25) (layer F.Cu) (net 1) (status 30))
 (segment (start 106.6 102.6) (end 106.6 104.6) (width 0.25) (layer F.Cu) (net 1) (status 30))
 (segment (start 106.6 108.2) (end 106.6 110.2) (width 0.25) (layer F.Cu) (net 1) (status 30))
 (via (at 106.6 104.6) (size 0.8) (drill 0.4) (layers F.Cu B.Cu) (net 1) (status 30))
 (segment (start 107.445 103.755) (end 106.6 104.6) (width 0.25) (layer B.Cu) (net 1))
 (segment (start 107.95 103.755) (end 107.445 103.755) (width 0.25) (layer B.Cu) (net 1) (status 10))
 (segment (start 110.6 102.6) (end 110.6 104.6) (width 0.25) (layer F.Cu) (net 4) (status 30))
 (segment (start 110.6 110.2) (end 110.6 108.2) (width 0.25) (layer F.Cu) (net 4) (status 30))
 (segment (start 110.6 108.6) (end 110.6 110.6) (width 0.25) (layer F.Cu) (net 4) (status 30))
 (segment (start 110.6 106.6) (end 110.6 108.6) (width 0.25) (layer F.Cu) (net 4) (status 30))
 (segment (start 110.6 104.6) (end 110.6 106.6) (width 0.25) (layer F.Cu) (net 4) (status 30))
 (segment (start 110.6 108.2) (end 110.6 106.2) (width 0.25) (layer F.Cu) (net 4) (status 30))
 (via (at 110.6 104.6) (size 0.8) (drill 0.4) (layers F.Cu B.Cu) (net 4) (status 30))
 (segment (start 111.445 103.755) (end 110.6 104.6) (width 0.25) (layer B.Cu) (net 4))
 (segment (start 113.03 103.755) (end 111.445 103.755) (width 0.25) (layer B.Cu) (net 4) (status 10))
 (segment (start 114.6 108.6) (end 114.6 110.6) (width 0.25) (layer F.Cu) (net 3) (status 30))
 (segment (start 114.6 106.6) (end 114.6 108.6) (width 0.25) (layer F.Cu) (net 3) (status 30))
 (segment (start 114.6 108.2) (end 114.6 110.2) (width 0.25) (layer F.Cu) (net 3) (status 30))
 (segment (start 114.6 106.2) (end 114.6 108.2) (width 0.25) (layer F.Cu) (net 3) (status 30))
 (segment (start 114.6 104.6) (end 114.6 106.6) (width 0.25) (layer F.Cu) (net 3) (status 30))
 (segment (start 114.6 102.6) (end 114.6 104.6) (width 0.25) (layer F.Cu) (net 3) (status 30))
 (via (at 114.6 104.6) (size 0.8) (drill 0.4) (layers F.Cu B.Cu) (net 3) (status 30))
 (segment (start 115.445 103.755) (end 114.6 104.6) (width 0.25) (layer B.Cu) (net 3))
 (segment (start 118.11 103.755) (end 115.445 103.755) (width 0.25) (layer B.Cu) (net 3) (status 10))
 (segment (start 104.6 108.6) (end 104.6 110.6) (width 0.25) (layer F.Cu) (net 10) (status 30))
 (segment (start 104.6 106.6) (end 104.6 108.6) (width 0.25) (layer F.Cu) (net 10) (status 30))
 (segment (start 104.6 104.6) (end 104.6 106.6) (width 0.25) (layer F.Cu) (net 10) (status 30))
 (segment (start 104.6 107) (end 104.6 105) (width 0.25) (layer F.Cu) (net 10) (status 30))
 (segment (start 104.6 109) (end 104.6 107) (width 0.25) (layer F.Cu) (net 10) (status 30))
 (segment (start 104.6 102.6) (end 104.6 104.6) (width 0.25) (layer F.Cu) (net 10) (status 30))
 (segment (start 104.6 105) (end 104.6 103) (width 0.25) (layer F.Cu) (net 10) (status 30))
 (via (at 104.6 106.6) (size 0.8) (drill 0.4) (layers F.Cu B.Cu) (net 10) (status 30))
 (segment (start 105.065 107.065) (end 104.6 106.6) (width 0.25) (layer B.Cu) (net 10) (status 10))
 (segment (start 105.41 107.065) (end 105.065 107.065) (width 0.25) (layer B.Cu) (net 10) (status 30))
 (segment (start 108.6 105) (end 108.6 103) (width 0.25) (layer F.Cu) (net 11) (status 30))
 (segment (start 108.6 107) (end 108.6 105) (width 0.25) (layer F.Cu) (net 11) (status 30))
 (segment (start 108.6 109) (end 108.6 107) (width 0.25) (layer F.Cu) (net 11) (status 30))
 (segment (start 108.6 108.6) (end 108.6 110.6) (width 0.25) (layer F.Cu) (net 11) (status 30))
 (segment (start 108.6 106.6) (end 108.6 108.6) (width 0.25) (layer F.Cu) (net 11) (status 30))
 (segment (start 108.6 104.6) (end 108.6 106.6) (width 0.25) (layer F.Cu) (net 11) (status 30))
 (segment (start 108.6 102.6) (end 108.6 104.6) (width 0.25) (layer F.Cu) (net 11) (status 30))
 (via (at 108.6 106.6) (size 0.8) (drill 0.4) (layers F.Cu B.Cu) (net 11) (status 30))
 (segment (start 109.065 107.065) (end 108.6 106.6) (width 0.25) (layer B.Cu) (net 11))
 (segment (start 110.49 107.065) (end 109.065 107.065) (width 0.25) (layer B.Cu) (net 11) (status 10))
 (segment (start 112.6 107) (end 112.6 105) (width 0.25) (layer F.Cu) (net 2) (status 30))
 (segment (start 112.6 104.6) (end 112.6 106.6) (width 0.25) (layer F.Cu) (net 2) (status 30))
 (segment (start 112.6 102.6) (end 112.6 104.6) (width 0.25) (layer F.Cu) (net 2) (status 30))
 (segment (start 112.6 105) (end 112.6 103) (width 0.25) (layer F.Cu) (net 2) (status 30))
 (segment (start 112.6 109) (end 112.6 107) (width 0.25) (layer F.Cu) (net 2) (status 30))
 (segment (start 112.6 108.6) (end 112.6 110.6) (width 0.25) (layer F.Cu) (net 2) (status 30))
 (segment (start 112.6 106.6) (end 112.6 108.6) (width 0.25) (layer F.Cu) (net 2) (status 30))
 (via (at 112.6 106.6) (size 0.8) (drill 0.4) (layers F.Cu B.Cu) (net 2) (status 30))
 (segment (start 113.065 107.065) (end 112.6 106.6) (width 0.25) (layer B.Cu) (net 2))
 (segment (start 115.57 107.065) (end 113.065 107.065) (width 0.25) (layer B.Cu) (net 2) (status 10))
 (segment (start 116.6 106.6) (end 116.6 108.6) (width 0.25) (layer F.Cu) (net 5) (status 30))
 (segment (start 116.6 104.6) (end 116.6 106.6) (width 0.25) (layer F.Cu) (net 5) (status 30))
 (segment (start 116.6 108.6) (end 116.6 110.6) (width 0.25) (layer F.Cu) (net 5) (status 30))
 (segment (start 116.6 109) (end 116.6 107) (width 0.25) (layer F.Cu) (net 5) (status 30))
 (segment (start 116.6 102.6) (end 116.6 104.6) (width 0.25) (layer F.Cu) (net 5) (status 30))
 (segment (start 116.6 105) (end 116.6 103) (width 0.25) (layer F.Cu) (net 5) (status 30))
 (segment (start 116.6 107) (end 116.6 105) (width 0.25) (layer F.Cu) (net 5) (status 30))
 (via (at 116.6 104.6) (size 0.8) (drill 0.4) (layers F.Cu B.Cu) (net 5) (status 30))
 (segment (start 119.065 107.065) (end 116.6 104.6) (width 0.25) (layer B.Cu) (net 5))
 (segment (start 120.65 107.065) (end 119.065 107.065) (width 0.25) (layer B.Cu) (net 5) (status 10)))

